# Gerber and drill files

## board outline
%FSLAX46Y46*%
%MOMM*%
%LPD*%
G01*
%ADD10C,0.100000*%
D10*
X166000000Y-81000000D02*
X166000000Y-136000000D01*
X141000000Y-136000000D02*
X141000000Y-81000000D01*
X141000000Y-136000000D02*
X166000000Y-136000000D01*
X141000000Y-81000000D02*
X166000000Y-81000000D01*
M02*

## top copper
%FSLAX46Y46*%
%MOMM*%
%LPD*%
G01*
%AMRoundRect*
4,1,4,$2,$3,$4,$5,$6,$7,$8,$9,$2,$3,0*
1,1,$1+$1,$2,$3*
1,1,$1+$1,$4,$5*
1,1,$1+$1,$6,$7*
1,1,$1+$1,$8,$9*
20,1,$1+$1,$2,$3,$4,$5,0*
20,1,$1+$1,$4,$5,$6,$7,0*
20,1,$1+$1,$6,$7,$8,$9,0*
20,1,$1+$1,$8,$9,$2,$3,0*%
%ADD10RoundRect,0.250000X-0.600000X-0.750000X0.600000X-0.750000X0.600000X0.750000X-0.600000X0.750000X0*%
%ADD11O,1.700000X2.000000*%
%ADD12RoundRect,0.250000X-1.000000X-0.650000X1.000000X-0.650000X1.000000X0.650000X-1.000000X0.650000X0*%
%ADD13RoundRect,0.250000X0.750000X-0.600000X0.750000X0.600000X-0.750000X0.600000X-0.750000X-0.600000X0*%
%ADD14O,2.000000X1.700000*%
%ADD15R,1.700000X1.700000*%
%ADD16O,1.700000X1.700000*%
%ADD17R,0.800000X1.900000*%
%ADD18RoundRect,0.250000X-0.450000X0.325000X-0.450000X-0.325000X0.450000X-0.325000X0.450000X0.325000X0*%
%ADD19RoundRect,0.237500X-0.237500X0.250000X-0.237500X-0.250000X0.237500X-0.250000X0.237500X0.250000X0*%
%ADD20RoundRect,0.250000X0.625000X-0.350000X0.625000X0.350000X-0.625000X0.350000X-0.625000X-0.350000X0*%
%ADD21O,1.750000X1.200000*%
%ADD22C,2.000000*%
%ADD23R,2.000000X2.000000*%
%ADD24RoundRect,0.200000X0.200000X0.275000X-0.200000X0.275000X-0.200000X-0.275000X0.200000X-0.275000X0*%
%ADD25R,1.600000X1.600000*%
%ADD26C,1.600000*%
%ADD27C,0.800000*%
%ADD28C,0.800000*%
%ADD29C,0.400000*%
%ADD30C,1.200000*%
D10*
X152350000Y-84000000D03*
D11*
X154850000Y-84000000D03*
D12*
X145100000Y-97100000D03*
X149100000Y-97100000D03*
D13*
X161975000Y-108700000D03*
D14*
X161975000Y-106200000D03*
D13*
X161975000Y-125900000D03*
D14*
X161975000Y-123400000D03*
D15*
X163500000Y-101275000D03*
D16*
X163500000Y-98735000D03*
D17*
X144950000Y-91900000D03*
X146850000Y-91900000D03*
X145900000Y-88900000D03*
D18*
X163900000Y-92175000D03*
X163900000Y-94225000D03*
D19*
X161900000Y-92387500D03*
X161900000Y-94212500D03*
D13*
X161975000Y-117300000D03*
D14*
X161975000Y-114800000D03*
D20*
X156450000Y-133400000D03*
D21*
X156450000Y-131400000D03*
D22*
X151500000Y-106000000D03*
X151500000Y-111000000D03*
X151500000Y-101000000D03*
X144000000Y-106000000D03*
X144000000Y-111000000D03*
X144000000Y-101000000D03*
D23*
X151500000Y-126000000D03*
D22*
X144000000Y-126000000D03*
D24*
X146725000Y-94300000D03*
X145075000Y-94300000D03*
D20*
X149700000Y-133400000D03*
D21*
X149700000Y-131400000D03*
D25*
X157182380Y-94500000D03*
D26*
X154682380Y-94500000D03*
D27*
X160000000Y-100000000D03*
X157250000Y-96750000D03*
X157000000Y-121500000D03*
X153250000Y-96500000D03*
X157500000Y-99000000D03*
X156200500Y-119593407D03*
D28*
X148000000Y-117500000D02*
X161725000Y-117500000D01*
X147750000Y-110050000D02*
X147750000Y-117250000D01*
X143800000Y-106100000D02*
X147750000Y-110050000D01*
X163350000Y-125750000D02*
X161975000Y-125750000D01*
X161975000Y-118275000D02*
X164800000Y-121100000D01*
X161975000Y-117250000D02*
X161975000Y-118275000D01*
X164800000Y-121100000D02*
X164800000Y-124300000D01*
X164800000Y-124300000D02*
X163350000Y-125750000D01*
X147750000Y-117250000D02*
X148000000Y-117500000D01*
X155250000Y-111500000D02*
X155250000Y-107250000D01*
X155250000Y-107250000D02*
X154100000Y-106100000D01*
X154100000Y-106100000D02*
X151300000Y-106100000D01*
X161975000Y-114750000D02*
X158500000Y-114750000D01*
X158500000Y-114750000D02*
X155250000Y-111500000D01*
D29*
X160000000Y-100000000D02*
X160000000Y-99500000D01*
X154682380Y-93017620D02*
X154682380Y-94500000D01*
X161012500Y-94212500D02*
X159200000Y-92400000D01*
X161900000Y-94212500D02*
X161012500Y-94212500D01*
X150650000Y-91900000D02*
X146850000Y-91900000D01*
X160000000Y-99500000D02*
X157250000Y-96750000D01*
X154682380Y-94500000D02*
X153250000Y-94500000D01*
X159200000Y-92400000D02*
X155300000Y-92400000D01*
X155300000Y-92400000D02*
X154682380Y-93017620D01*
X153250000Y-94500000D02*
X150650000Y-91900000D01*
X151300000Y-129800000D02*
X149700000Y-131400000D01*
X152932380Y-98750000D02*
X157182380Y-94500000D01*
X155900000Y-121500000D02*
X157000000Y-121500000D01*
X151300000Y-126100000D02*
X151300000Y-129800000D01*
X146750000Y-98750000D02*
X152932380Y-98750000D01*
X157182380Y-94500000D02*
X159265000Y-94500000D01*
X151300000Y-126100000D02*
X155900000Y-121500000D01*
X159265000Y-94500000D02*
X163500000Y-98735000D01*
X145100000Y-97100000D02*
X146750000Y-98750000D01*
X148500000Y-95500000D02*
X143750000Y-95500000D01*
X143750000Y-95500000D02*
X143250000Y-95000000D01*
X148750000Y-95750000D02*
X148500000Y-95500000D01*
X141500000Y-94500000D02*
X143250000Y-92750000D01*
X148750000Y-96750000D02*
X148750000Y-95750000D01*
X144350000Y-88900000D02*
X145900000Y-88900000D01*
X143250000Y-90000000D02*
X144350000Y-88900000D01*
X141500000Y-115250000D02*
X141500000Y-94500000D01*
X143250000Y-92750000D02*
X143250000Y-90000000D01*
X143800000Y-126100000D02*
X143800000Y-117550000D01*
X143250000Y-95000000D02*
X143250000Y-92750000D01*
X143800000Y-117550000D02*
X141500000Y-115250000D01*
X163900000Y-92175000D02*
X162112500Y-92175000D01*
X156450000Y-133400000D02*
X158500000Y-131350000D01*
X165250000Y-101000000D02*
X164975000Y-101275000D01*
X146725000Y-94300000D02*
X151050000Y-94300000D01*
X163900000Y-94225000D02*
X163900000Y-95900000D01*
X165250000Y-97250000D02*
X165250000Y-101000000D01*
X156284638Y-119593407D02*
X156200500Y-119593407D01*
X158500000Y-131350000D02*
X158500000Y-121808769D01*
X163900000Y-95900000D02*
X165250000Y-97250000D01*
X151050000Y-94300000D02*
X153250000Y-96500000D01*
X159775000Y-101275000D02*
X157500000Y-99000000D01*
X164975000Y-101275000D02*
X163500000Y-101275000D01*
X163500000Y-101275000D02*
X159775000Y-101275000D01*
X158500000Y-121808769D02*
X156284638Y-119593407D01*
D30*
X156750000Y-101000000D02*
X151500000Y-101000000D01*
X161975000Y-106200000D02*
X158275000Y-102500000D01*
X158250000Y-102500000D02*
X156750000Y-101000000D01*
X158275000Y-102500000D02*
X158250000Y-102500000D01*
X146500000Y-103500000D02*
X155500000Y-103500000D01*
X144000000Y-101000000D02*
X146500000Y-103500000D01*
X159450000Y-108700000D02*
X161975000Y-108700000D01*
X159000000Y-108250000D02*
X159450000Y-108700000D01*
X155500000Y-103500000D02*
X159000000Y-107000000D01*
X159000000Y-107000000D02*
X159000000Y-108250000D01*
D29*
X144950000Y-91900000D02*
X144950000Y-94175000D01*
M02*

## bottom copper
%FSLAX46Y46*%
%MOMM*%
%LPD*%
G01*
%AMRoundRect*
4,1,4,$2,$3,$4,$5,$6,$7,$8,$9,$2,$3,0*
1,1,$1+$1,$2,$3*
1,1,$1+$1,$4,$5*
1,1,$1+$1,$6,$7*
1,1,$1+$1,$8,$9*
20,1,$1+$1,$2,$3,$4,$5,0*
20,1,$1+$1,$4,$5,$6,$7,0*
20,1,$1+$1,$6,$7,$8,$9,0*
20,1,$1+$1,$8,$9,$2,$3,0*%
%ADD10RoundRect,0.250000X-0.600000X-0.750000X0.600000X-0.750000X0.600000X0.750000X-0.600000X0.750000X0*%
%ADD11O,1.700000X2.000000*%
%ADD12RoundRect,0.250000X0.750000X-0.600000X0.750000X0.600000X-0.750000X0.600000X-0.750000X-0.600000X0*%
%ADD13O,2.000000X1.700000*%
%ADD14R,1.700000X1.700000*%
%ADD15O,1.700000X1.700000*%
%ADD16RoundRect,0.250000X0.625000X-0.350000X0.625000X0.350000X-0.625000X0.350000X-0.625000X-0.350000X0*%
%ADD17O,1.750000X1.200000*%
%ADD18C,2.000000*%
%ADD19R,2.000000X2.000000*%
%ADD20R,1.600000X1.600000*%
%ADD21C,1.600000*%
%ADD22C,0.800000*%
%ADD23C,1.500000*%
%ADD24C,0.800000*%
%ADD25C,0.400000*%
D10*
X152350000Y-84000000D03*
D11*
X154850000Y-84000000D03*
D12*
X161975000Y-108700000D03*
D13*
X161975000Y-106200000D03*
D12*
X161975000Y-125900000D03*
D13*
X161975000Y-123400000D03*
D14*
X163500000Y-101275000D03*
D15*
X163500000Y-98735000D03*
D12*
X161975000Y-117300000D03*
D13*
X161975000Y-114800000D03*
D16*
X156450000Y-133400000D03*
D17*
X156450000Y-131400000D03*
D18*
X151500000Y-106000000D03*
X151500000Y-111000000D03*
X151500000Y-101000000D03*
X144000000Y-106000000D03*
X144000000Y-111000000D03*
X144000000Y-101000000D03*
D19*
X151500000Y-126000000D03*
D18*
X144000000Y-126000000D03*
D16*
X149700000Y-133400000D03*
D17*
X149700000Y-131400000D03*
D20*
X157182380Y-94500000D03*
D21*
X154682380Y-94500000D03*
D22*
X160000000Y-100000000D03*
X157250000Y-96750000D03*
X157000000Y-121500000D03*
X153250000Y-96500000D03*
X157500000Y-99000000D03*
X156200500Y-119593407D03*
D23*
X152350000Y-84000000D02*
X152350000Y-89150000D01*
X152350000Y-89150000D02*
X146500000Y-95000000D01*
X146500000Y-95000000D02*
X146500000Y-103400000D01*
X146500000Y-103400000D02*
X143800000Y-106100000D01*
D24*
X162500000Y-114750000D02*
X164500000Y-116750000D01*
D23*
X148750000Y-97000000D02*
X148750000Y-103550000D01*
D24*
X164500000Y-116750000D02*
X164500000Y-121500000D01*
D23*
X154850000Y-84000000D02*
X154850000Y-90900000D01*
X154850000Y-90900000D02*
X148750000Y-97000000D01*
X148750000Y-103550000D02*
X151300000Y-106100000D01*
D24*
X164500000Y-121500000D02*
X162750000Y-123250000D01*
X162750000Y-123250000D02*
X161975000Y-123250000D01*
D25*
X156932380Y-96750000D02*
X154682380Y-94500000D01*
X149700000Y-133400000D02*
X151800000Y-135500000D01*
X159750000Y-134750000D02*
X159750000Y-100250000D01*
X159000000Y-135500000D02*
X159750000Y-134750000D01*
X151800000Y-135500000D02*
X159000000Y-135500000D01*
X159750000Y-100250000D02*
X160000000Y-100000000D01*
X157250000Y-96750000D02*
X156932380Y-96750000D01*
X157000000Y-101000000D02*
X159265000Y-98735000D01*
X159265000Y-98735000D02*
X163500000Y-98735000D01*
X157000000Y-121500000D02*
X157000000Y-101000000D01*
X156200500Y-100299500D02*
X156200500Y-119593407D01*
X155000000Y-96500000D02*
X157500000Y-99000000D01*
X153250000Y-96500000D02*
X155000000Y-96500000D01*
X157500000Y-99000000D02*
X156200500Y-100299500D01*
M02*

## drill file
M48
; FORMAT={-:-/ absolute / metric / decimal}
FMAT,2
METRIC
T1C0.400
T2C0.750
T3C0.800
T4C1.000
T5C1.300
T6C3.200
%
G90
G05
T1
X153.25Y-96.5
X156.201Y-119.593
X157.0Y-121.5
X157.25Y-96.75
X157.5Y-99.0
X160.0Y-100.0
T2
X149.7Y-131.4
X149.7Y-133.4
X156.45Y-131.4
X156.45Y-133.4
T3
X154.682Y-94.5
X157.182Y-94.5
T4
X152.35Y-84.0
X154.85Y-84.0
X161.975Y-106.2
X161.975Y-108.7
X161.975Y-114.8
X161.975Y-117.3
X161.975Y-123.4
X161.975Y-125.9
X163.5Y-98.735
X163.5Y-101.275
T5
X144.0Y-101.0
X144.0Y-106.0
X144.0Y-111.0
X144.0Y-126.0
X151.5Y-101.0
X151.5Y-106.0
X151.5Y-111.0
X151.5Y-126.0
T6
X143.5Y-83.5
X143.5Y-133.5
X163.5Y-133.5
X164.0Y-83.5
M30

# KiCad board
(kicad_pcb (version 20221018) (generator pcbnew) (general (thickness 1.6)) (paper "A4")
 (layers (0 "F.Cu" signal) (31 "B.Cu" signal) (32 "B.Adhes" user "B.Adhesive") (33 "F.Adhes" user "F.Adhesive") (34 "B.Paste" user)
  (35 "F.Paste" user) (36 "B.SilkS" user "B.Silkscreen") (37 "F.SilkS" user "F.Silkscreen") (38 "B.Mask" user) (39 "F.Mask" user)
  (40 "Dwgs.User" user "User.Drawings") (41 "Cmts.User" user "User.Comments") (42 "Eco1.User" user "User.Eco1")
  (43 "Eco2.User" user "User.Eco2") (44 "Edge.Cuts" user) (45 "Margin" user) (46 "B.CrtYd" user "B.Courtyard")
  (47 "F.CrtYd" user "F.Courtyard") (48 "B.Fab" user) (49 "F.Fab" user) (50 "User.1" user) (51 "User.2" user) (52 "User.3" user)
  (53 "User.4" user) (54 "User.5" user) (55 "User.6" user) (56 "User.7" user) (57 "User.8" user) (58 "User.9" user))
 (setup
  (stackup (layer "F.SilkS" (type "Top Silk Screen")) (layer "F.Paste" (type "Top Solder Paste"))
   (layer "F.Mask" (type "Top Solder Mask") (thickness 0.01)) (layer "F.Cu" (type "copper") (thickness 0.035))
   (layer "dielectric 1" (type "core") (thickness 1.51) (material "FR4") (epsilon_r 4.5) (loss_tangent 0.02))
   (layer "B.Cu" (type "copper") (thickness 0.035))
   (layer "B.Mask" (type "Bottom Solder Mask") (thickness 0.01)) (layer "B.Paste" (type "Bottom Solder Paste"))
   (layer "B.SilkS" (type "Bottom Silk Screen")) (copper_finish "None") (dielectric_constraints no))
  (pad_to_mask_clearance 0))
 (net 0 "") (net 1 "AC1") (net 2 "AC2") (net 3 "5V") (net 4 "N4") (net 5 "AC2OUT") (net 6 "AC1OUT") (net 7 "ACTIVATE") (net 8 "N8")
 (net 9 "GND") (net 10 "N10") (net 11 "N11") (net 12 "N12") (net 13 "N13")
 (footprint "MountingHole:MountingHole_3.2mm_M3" (layer "F.Cu") (at 163.5 133.5)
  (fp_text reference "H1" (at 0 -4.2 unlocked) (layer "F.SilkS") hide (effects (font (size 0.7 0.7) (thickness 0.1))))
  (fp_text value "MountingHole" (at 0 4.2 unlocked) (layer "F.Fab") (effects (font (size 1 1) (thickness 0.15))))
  (pad "" np_thru_hole circle (at 0 0) (size 3.2 3.2) (drill 3.2) (layers "*.Cu" "*.Mask")))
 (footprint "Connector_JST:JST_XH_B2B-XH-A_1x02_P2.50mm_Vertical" (layer "F.Cu") (at 152.35 84)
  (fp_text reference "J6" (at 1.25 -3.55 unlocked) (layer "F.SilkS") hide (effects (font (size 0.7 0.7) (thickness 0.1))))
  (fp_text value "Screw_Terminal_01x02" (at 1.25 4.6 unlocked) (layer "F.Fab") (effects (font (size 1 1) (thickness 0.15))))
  (pad "1" thru_hole roundrect (at 0 0) (size 1.7 2) (drill 1) (layers "*.Cu" "*.Mask") (roundrect_rratio 0.147059) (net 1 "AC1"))
  (pad "2" thru_hole oval (at 2.5 0) (size 1.7 2) (drill 1) (layers "*.Cu" "*.Mask") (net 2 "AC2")))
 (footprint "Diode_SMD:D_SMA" (layer "F.Cu") (at 147.1 97.1)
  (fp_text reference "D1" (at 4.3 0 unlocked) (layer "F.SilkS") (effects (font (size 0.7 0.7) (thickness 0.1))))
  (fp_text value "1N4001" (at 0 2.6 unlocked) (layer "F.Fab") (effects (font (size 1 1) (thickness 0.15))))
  (pad "1" smd roundrect (at -2 0) (size 2.5 1.8) (layers "F.Cu" "F.Paste" "F.Mask") (roundrect_rratio 0.1388888889) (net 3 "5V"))
  (pad "2" smd roundrect (at 2 0) (size 2.5 1.8) (layers "F.Cu" "F.Paste" "F.Mask") (roundrect_rratio 0.1388888889) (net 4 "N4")))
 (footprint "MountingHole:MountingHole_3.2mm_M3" (layer "F.Cu") (at 164 83.5)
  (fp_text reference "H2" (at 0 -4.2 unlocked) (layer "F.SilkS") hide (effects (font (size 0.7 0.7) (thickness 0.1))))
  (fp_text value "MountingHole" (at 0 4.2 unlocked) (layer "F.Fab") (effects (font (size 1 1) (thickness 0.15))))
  (pad "" np_thru_hole circle (at 0 0) (size 3.2 3.2) (drill 3.2) (layers "*.Cu" "*.Mask")))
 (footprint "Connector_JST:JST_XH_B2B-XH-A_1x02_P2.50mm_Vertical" (layer "F.Cu") (at 161.975 108.7 90)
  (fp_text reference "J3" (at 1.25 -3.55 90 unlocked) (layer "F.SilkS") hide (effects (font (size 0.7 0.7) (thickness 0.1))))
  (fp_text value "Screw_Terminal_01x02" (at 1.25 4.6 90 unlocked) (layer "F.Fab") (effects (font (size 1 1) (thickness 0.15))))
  (pad "1" thru_hole roundrect (at 0 0 90) (size 1.7 2) (drill 1) (layers "*.Cu" "*.Mask") (roundrect_rratio 0.147059) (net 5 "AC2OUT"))
  (pad "2" thru_hole oval (at 2.5 0 90) (size 1.7 2) (drill 1) (layers "*.Cu" "*.Mask") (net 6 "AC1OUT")))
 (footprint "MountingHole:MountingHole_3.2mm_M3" (layer "F.Cu") (at 143.5 83.5)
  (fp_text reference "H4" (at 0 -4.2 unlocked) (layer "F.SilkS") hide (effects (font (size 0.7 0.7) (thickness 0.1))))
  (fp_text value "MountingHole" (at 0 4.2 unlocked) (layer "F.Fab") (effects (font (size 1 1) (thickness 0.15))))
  (pad "" np_thru_hole circle (at 0 0) (size 3.2 3.2) (drill 3.2) (layers "*.Cu" "*.Mask")))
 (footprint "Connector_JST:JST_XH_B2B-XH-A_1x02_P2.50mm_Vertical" (layer "F.Cu") (at 161.975 125.9 90)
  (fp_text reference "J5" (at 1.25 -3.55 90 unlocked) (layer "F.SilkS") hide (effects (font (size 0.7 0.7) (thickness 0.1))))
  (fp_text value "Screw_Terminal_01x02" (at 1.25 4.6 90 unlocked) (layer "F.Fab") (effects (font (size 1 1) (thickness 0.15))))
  (pad "1" thru_hole roundrect (at 0 0 90) (size 1.7 2) (drill 1) (layers "*.Cu" "*.Mask") (roundrect_rratio 0.147059) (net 1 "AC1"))
  (pad "2" thru_hole oval (at 2.5 0 90) (size 1.7 2) (drill 1) (layers "*.Cu" "*.Mask") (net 2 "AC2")))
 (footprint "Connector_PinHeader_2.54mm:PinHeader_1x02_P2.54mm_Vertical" (layer "F.Cu") (at 163.5 101.275 180)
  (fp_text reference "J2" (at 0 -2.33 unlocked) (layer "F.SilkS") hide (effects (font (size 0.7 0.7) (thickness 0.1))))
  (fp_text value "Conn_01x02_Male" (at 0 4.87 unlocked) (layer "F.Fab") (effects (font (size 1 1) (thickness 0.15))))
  (pad "1" thru_hole rect (at 0 0 180) (size 1.7 1.7) (drill 1) (layers "*.Cu" "*.Mask") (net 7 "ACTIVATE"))
  (pad "2" thru_hole oval (at 0 2.54 180) (size 1.7 1.7) (drill 1) (layers "*.Cu" "*.Mask") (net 3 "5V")))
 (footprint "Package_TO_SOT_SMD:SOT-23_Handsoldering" (layer "F.Cu") (at 145.9 90.4 90)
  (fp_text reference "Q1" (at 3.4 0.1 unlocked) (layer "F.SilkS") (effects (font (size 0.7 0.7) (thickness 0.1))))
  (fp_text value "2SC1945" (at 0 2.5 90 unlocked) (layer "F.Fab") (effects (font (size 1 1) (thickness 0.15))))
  (pad "1" smd rect (at -1.5 -0.95 90) (size 1.9 0.8) (layers "F.Cu" "F.Paste" "F.Mask") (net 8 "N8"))
  (pad "2" smd rect (at -1.5 0.95 90) (size 1.9 0.8) (layers "F.Cu" "F.Paste" "F.Mask") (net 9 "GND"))
  (pad "3" smd rect (at 1.5 0 90) (size 1.9 0.8) (layers "F.Cu" "F.Paste" "F.Mask") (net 4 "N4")))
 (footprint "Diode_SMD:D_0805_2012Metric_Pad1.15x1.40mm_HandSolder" (layer "F.Cu") (at 163.9 93.2 -90)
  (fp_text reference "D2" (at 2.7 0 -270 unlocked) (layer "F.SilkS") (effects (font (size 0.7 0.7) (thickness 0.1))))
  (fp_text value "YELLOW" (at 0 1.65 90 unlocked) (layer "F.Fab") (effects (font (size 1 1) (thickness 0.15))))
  (pad "1" smd roundrect (at -1.025 0 270) (size 1.15 1.4) (layers "F.Cu" "F.Paste" "F.Mask") (roundrect_rratio 0.217391) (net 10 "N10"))
  (pad "2" smd roundrect (at 1.025 0 270) (size 1.15 1.4) (layers "F.Cu" "F.Paste" "F.Mask") (roundrect_rratio 0.217391) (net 7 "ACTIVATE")))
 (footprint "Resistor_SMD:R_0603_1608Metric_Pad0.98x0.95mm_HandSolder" (layer "F.Cu") (at 161.9 93.3 -90)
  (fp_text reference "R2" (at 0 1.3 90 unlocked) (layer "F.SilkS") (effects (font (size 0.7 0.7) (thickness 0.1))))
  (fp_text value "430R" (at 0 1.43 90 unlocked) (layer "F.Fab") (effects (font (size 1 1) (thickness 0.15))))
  (pad "1" smd roundrect (at -0.9125 0 270) (size 0.975 0.95) (layers "F.Cu" "F.Paste" "F.Mask") (roundrect_rratio 0.25) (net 10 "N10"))
  (pad "2" smd roundrect (at 0.9125 0 270) (size 0.975 0.95) (layers "F.Cu" "F.Paste" "F.Mask") (roundrect_rratio 0.25) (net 9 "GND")))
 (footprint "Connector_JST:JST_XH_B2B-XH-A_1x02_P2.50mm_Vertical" (layer "F.Cu") (at 161.975 117.3 90)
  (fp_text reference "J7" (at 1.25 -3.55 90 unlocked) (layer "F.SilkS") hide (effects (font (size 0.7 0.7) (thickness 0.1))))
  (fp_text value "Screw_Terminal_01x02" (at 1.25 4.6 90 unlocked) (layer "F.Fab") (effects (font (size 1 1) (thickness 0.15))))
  (pad "1" thru_hole roundrect (at 0 0 90) (size 1.7 2) (drill 1) (layers "*.Cu" "*.Mask") (roundrect_rratio 0.147059) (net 1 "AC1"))
  (pad "2" thru_hole oval (at 2.5 0 90) (size 1.7 2) (drill 1) (layers "*.Cu" "*.Mask") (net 2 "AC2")))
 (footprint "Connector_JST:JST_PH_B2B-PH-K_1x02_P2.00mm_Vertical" (layer "F.Cu") (at 156.45 133.4 90)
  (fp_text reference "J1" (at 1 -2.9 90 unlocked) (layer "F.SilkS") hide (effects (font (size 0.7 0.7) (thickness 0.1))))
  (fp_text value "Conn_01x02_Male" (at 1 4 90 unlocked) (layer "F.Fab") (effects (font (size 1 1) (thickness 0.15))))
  (pad "1" thru_hole roundrect (at 0 0 90) (size 1.2 1.75) (drill 0.75) (layers "*.Cu" "*.Mask") (roundrect_rratio 0.208333)
   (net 7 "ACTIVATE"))
  (pad "2" thru_hole oval (at 2 0 90) (size 1.2 1.75) (drill 0.75) (layers "*.Cu" "*.Mask") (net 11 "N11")))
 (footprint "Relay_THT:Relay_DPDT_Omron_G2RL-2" (layer "F.Cu") (at 151.5 126 180)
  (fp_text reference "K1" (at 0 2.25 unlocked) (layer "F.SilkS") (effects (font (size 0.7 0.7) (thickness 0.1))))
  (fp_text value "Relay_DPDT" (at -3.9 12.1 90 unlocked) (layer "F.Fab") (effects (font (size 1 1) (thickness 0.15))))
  (pad "11" thru_hole circle (at 0 20 180) (size 2 2) (drill 1.3) (layers "*.Cu" "*.Mask") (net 2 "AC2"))
  (pad "12" thru_hole circle (at 0 15 180) (size 2 2) (drill 1.3) (layers "*.Cu" "*.Mask") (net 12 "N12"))
  (pad "14" thru_hole circle (at 0 25 180) (size 2 2) (drill 1.3) (layers "*.Cu" "*.Mask") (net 6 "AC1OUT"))
  (pad "21" thru_hole circle (at 7.5 20 180) (size 2 2) (drill 1.3) (layers "*.Cu" "*.Mask") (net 1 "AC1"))
  (pad "22" thru_hole circle (at 7.5 15 180) (size 2 2) (drill 1.3) (layers "*.Cu" "*.Mask") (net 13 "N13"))
  (pad "24" thru_hole circle (at 7.5 25 180) (size 2 2) (drill 1.3) (layers "*.Cu" "*.Mask") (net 5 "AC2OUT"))
  (pad "A1" thru_hole rect (at 0 0 180) (size 2 2) (drill 1.3) (layers "*.Cu" "*.Mask") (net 3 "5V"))
  (pad "A2" thru_hole circle (at 7.5 0 180) (size 2 2) (drill 1.3) (layers "*.Cu" "*.Mask") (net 4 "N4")))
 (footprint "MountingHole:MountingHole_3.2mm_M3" (layer "F.Cu") (at 143.5 133.5)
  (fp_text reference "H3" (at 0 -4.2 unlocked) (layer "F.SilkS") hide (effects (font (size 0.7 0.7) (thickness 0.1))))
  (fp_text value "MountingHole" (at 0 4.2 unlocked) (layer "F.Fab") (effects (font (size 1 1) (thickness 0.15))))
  (pad "" np_thru_hole circle (at 0 0) (size 3.2 3.2) (drill 3.2) (layers "*.Cu" "*.Mask")))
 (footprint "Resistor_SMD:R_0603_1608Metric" (layer "F.Cu") (at 145.9 94.3 180)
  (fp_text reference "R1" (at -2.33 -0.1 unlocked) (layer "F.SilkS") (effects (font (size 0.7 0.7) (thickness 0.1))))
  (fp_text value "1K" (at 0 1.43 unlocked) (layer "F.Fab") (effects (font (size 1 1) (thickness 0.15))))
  (pad "1" smd roundrect (at -0.825 0 180) (size 0.8 0.95) (layers "F.Cu" "F.Paste" "F.Mask") (roundrect_rratio 0.25) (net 7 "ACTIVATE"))
  (pad "2" smd roundrect (at 0.825 0 180) (size 0.8 0.95) (layers "F.Cu" "F.Paste" "F.Mask") (roundrect_rratio 0.25) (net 8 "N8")))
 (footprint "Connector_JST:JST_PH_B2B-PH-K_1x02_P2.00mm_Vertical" (layer "F.Cu") (at 149.7 133.4 90)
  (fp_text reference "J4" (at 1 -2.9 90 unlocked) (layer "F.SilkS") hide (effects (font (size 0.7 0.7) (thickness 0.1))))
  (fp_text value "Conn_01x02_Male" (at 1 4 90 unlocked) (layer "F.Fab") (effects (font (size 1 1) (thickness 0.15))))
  (pad "1" thru_hole roundrect (at 0 0 90) (size 1.2 1.75) (drill 0.75) (layers "*.Cu" "*.Mask") (roundrect_rratio 0.208333) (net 9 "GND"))
  (pad "2" thru_hole oval (at 2 0 90) (size 1.2 1.75) (drill 0.75) (layers "*.Cu" "*.Mask") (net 3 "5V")))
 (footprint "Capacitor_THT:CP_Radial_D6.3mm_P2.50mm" (layer "F.Cu") (at 157.18238 94.5 180)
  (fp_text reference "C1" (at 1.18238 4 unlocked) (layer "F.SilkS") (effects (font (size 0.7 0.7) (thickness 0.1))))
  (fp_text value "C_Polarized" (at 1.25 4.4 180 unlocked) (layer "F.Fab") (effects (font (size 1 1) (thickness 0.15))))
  (pad "1" thru_hole rect (at 0 0 180) (size 1.6 1.6) (drill 0.8) (layers "*.Cu" "*.Mask") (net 3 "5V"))
  (pad "2" thru_hole circle (at 2.5 0 180) (size 1.6 1.6) (drill 0.8) (layers "*.Cu" "*.Mask") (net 9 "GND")))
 (gr_line (start 166 81) (end 166 136) (stroke (width 0.1) (type solid)) (layer "Edge.Cuts"))
 (gr_line (start 141 136) (end 141 81) (stroke (width 0.1) (type solid)) (layer "Edge.Cuts"))
 (gr_line (start 141 136) (end 166 136) (stroke (width 0.1) (type solid)) (layer "Edge.Cuts"))
 (gr_line (start 141 81) (end 166 81) (stroke (width 0.1) (type solid)) (layer "Edge.Cuts"))
 (segment (start 148 117.5) (end 161.725 117.5) (width 0.8) (layer "F.Cu") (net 1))
 (segment (start 147.75 110.05) (end 147.75 117.25) (width 0.8) (layer "F.Cu") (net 1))
 (segment (start 143.8 106.1) (end 147.75 110.05) (width 0.8) (layer "F.Cu") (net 1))
 (segment (start 163.35 125.75) (end 161.975 125.75) (width 0.8) (layer "F.Cu") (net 1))
 (segment (start 161.975 118.275) (end 164.8 121.1) (width 0.8) (layer "F.Cu") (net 1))
 (segment (start 161.975 117.25) (end 161.975 118.275) (width 0.8) (layer "F.Cu") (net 1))
 (segment (start 164.8 121.1) (end 164.8 124.3) (width 0.8) (layer "F.Cu") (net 1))
 (segment (start 164.8 124.3) (end 163.35 125.75) (width 0.8) (layer "F.Cu") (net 1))
 (segment (start 147.75 117.25) (end 148 117.5) (width 0.8) (layer "F.Cu") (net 1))
 (segment (start 152.35 84) (end 152.35 89.15) (width 1.5) (layer "B.Cu") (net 1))
 (segment (start 152.35 89.15) (end 146.5 95) (width 1.5) (layer "B.Cu") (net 1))
 (segment (start 146.5 95) (end 146.5 103.4) (width 1.5) (layer "B.Cu") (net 1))
 (segment (start 146.5 103.4) (end 143.8 106.1) (width 1.5) (layer "B.Cu") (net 1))
 (segment (start 155.25 111.5) (end 155.25 107.25) (width 0.8) (layer "F.Cu") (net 2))
 (segment (start 155.25 107.25) (end 154.1 106.1) (width 0.8) (layer "F.Cu") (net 2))
 (segment (start 154.1 106.1) (end 151.3 106.1) (width 0.8) (layer "F.Cu") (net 2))
 (segment (start 161.975 114.75) (end 158.5 114.75) (width 0.8) (layer "F.Cu") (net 2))
 (segment (start 158.5 114.75) (end 155.25 111.5) (width 0.8) (layer "F.Cu") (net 2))
 (segment (start 162.5 114.75) (end 164.5 116.75) (width 0.8) (layer "B.Cu") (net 2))
 (segment (start 148.75 97) (end 148.75 103.55) (width 1.5) (layer "B.Cu") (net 2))
 (segment (start 164.5 116.75) (end 164.5 121.5) (width 0.8) (layer "B.Cu") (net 2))
 (segment (start 154.85 84) (end 154.85 90.9) (width 1.5) (layer "B.Cu") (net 2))
 (segment (start 154.85 90.9) (end 148.75 97) (width 1.5) (layer "B.Cu") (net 2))
 (segment (start 148.75 103.55) (end 151.3 106.1) (width 1.5) (layer "B.Cu") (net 2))
 (segment (start 164.5 121.5) (end 162.75 123.25) (width 0.8) (layer "B.Cu") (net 2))
 (segment (start 162.75 123.25) (end 161.975 123.25) (width 0.8) (layer "B.Cu") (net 2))
 (segment (start 160 100) (end 160 99.5) (width 0.4) (layer "F.Cu") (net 9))
 (segment (start 154.68238 93.01762) (end 154.68238 94.5) (width 0.4) (layer "F.Cu") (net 9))
 (segment (start 161.0125 94.2125) (end 159.2 92.4) (width 0.4) (layer "F.Cu") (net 9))
 (segment (start 161.9 94.2125) (end 161.0125 94.2125) (width 0.4) (layer "F.Cu") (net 9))
 (segment (start 150.65 91.9) (end 146.85 91.9) (width 0.4) (layer "F.Cu") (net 9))
 (segment (start 160 99.5) (end 157.25 96.75) (width 0.4) (layer "F.Cu") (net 9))
 (segment (start 154.68238 94.5) (end 153.25 94.5) (width 0.4) (layer "F.Cu") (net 9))
 (segment (start 159.2 92.4) (end 155.3 92.4) (width 0.4) (layer "F.Cu") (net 9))
 (segment (start 155.3 92.4) (end 154.68238 93.01762) (width 0.4) (layer "F.Cu") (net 9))
 (segment (start 153.25 94.5) (end 150.65 91.9) (width 0.4) (layer "F.Cu") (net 9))
 (via (at 160 100) (size 0.8) (drill 0.4) (layers "F.Cu" "B.Cu") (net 9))
 (via (at 157.25 96.75) (size 0.8) (drill 0.4) (layers "F.Cu" "B.Cu") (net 9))
 (segment (start 156.93238 96.75) (end 154.68238 94.5) (width 0.4) (layer "B.Cu") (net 9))
 (segment (start 149.7 133.4) (end 151.8 135.5) (width 0.4) (layer "B.Cu") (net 9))
 (segment (start 159.75 134.75) (end 159.75 100.25) (width 0.4) (layer "B.Cu") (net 9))
 (segment (start 159 135.5) (end 159.75 134.75) (width 0.4) (layer "B.Cu") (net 9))
 (segment (start 151.8 135.5) (end 159 135.5) (width 0.4) (layer "B.Cu") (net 9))
 (segment (start 159.75 100.25) (end 160 100) (width 0.4) (layer "B.Cu") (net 9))
 (segment (start 157.25 96.75) (end 156.93238 96.75) (width 0.4) (layer "B.Cu") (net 9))
 (segment (start 151.3 129.8) (end 149.7 131.4) (width 0.4) (layer "F.Cu") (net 3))
 (segment (start 152.93238 98.75) (end 157.18238 94.5) (width 0.4) (layer "F.Cu") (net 3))
 (segment (start 155.9 121.5) (end 157 121.5) (width 0.4) (layer "F.Cu") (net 3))
 (segment (start 151.3 126.1) (end 151.3 129.8) (width 0.4) (layer "F.Cu") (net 3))
 (segment (start 146.75 98.75) (end 152.93238 98.75) (width 0.4) (layer "F.Cu") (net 3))
 (segment (start 157.18238 94.5) (end 159.265 94.5) (width 0.4) (layer "F.Cu") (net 3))
 (segment (start 151.3 126.1) (end 155.9 121.5) (width 0.4) (layer "F.Cu") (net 3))
 (segment (start 159.265 94.5) (end 163.5 98.735) (width 0.4) (layer "F.Cu") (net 3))
 (segment (start 145.1 97.1) (end 146.75 98.75) (width 0.4) (layer "F.Cu") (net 3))
 (via (at 157 121.5) (size 0.8) (drill 0.4) (layers "F.Cu" "B.Cu") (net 3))
 (segment (start 157 101) (end 159.265 98.735) (width 0.4) (layer "B.Cu") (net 3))
 (segment (start 159.265 98.735) (end 163.5 98.735) (width 0.4) (layer "B.Cu") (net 3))
 (segment (start 157 121.5) (end 157 101) (width 0.4) (layer "B.Cu") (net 3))
 (segment (start 148.5 95.5) (end 143.75 95.5) (width 0.4) (layer "F.Cu") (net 4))
 (segment (start 143.75 95.5) (end 143.25 95) (width 0.4) (layer "F.Cu") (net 4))
 (segment (start 148.75 95.75) (end 148.5 95.5) (width 0.4) (layer "F.Cu") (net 4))
 (segment (start 141.5 94.5) (end 143.25 92.75) (width 0.4) (layer "F.Cu") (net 4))
 (segment (start 148.75 96.75) (end 148.75 95.75) (width 0.4) (layer "F.Cu") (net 4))
 (segment (start 144.35 88.9) (end 145.9 88.9) (width 0.4) (layer "F.Cu") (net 4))
 (segment (start 143.25 90) (end 144.35 88.9) (width 0.4) (layer "F.Cu") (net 4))
 (segment (start 141.5 115.25) (end 141.5 94.5) (width 0.4) (layer "F.Cu") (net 4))
 (segment (start 143.25 92.75) (end 143.25 90) (width 0.4) (layer "F.Cu") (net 4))
 (segment (start 143.8 126.1) (end 143.8 117.55) (width 0.4) (layer "F.Cu") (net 4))
 (segment (start 143.25 95) (end 143.25 92.75) (width 0.4) (layer "F.Cu") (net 4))
 (segment (start 143.8 117.55) (end 141.5 115.25) (width 0.4) (layer "F.Cu") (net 4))
 (segment (start 163.9 92.175) (end 162.1125 92.175) (width 0.4) (layer "F.Cu") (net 10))
 (segment (start 156.45 133.4) (end 158.5 131.35) (width 0.4) (layer "F.Cu") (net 7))
 (segment (start 165.25 101) (end 164.975 101.275) (width 0.4) (layer "F.Cu") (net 7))
 (segment (start 146.725 94.3) (end 151.05 94.3) (width 0.4) (layer "F.Cu") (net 7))
 (segment (start 163.9 94.225) (end 163.9 95.9) (width 0.4) (layer "F.Cu") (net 7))
 (segment (start 165.25 97.25) (end 165.25 101) (width 0.4) (layer "F.Cu") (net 7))
 (segment (start 156.284638 119.593407) (end 156.2005 119.593407) (width 0.4) (layer "F.Cu") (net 7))
 (segment (start 158.5 131.35) (end 158.5 121.808769) (width 0.4) (layer "F.Cu") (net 7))
 (segment (start 163.9 95.9) (end 165.25 97.25) (width 0.4) (layer "F.Cu") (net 7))
 (segment (start 151.05 94.3) (end 153.25 96.5) (width 0.4) (layer "F.Cu") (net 7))
 (segment (start 159.775 101.275) (end 157.5 99) (width 0.4) (layer "F.Cu") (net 7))
 (segment (start 164.975 101.275) (end 163.5 101.275) (width 0.4) (layer "F.Cu") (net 7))
 (segment (start 163.5 101.275) (end 159.775 101.275) (width 0.4) (layer "F.Cu") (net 7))
 (segment (start 158.5 121.808769) (end 156.284638 119.593407) (width 0.4) (layer "F.Cu") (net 7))
 (via (at 153.25 96.5) (size 0.8) (drill 0.4) (layers "F.Cu" "B.Cu") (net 7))
 (via (at 157.5 99) (size 0.8) (drill 0.4) (layers "F.Cu" "B.Cu") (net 7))
 (via (at 156.2005 119.593407) (size 0.8) (drill 0.4) (layers "F.Cu" "B.Cu") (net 7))
 (segment (start 156.2005 100.2995) (end 156.2005 119.593407) (width 0.4) (layer "B.Cu") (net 7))
 (segment (start 155 96.5) (end 157.5 99) (width 0.4) (layer "B.Cu") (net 7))
 (segment (start 153.25 96.5) (end 155 96.5) (width 0.4) (layer "B.Cu") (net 7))
 (segment (start 157.5 99) (end 156.2005 100.2995) (width 0.4) (layer "B.Cu") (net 7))
 (segment (start 156.75 101) (end 151.5 101) (width 1.2) (layer "F.Cu") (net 6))
 (segment (start 161.975 106.2) (end 158.275 102.5) (width 1.2) (layer "F.Cu") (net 6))
 (segment (start 158.25 102.5) (end 156.75 101) (width 1.2) (layer "F.Cu") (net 6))
 (segment (start 158.275 102.5) (end 158.25 102.5) (width 1.2) (layer "F.Cu") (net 6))
 (segment (start 146.5 103.5) (end 155.5 103.5) (width 1.2) (layer "F.Cu") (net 5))
 (segment (start 144 101) (end 146.5 103.5) (width 1.2) (layer "F.Cu") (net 5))
 (segment (start 159.45 108.7) (end 161.975 108.7) (width 1.2) (layer "F.Cu") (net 5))
 (segment (start 159 108.25) (end 159.45 108.7) (width 1.2) (layer "F.Cu") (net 5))
 (segment (start 155.5 103.5) (end 159 107) (width 1.2) (layer "F.Cu") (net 5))
 (segment (start 159 107) (end 159 108.25) (width 1.2) (layer "F.Cu") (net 5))
 (segment (start 144.95 91.9) (end 144.95 94.175) (width 0.4) (layer "F.Cu") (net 8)))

